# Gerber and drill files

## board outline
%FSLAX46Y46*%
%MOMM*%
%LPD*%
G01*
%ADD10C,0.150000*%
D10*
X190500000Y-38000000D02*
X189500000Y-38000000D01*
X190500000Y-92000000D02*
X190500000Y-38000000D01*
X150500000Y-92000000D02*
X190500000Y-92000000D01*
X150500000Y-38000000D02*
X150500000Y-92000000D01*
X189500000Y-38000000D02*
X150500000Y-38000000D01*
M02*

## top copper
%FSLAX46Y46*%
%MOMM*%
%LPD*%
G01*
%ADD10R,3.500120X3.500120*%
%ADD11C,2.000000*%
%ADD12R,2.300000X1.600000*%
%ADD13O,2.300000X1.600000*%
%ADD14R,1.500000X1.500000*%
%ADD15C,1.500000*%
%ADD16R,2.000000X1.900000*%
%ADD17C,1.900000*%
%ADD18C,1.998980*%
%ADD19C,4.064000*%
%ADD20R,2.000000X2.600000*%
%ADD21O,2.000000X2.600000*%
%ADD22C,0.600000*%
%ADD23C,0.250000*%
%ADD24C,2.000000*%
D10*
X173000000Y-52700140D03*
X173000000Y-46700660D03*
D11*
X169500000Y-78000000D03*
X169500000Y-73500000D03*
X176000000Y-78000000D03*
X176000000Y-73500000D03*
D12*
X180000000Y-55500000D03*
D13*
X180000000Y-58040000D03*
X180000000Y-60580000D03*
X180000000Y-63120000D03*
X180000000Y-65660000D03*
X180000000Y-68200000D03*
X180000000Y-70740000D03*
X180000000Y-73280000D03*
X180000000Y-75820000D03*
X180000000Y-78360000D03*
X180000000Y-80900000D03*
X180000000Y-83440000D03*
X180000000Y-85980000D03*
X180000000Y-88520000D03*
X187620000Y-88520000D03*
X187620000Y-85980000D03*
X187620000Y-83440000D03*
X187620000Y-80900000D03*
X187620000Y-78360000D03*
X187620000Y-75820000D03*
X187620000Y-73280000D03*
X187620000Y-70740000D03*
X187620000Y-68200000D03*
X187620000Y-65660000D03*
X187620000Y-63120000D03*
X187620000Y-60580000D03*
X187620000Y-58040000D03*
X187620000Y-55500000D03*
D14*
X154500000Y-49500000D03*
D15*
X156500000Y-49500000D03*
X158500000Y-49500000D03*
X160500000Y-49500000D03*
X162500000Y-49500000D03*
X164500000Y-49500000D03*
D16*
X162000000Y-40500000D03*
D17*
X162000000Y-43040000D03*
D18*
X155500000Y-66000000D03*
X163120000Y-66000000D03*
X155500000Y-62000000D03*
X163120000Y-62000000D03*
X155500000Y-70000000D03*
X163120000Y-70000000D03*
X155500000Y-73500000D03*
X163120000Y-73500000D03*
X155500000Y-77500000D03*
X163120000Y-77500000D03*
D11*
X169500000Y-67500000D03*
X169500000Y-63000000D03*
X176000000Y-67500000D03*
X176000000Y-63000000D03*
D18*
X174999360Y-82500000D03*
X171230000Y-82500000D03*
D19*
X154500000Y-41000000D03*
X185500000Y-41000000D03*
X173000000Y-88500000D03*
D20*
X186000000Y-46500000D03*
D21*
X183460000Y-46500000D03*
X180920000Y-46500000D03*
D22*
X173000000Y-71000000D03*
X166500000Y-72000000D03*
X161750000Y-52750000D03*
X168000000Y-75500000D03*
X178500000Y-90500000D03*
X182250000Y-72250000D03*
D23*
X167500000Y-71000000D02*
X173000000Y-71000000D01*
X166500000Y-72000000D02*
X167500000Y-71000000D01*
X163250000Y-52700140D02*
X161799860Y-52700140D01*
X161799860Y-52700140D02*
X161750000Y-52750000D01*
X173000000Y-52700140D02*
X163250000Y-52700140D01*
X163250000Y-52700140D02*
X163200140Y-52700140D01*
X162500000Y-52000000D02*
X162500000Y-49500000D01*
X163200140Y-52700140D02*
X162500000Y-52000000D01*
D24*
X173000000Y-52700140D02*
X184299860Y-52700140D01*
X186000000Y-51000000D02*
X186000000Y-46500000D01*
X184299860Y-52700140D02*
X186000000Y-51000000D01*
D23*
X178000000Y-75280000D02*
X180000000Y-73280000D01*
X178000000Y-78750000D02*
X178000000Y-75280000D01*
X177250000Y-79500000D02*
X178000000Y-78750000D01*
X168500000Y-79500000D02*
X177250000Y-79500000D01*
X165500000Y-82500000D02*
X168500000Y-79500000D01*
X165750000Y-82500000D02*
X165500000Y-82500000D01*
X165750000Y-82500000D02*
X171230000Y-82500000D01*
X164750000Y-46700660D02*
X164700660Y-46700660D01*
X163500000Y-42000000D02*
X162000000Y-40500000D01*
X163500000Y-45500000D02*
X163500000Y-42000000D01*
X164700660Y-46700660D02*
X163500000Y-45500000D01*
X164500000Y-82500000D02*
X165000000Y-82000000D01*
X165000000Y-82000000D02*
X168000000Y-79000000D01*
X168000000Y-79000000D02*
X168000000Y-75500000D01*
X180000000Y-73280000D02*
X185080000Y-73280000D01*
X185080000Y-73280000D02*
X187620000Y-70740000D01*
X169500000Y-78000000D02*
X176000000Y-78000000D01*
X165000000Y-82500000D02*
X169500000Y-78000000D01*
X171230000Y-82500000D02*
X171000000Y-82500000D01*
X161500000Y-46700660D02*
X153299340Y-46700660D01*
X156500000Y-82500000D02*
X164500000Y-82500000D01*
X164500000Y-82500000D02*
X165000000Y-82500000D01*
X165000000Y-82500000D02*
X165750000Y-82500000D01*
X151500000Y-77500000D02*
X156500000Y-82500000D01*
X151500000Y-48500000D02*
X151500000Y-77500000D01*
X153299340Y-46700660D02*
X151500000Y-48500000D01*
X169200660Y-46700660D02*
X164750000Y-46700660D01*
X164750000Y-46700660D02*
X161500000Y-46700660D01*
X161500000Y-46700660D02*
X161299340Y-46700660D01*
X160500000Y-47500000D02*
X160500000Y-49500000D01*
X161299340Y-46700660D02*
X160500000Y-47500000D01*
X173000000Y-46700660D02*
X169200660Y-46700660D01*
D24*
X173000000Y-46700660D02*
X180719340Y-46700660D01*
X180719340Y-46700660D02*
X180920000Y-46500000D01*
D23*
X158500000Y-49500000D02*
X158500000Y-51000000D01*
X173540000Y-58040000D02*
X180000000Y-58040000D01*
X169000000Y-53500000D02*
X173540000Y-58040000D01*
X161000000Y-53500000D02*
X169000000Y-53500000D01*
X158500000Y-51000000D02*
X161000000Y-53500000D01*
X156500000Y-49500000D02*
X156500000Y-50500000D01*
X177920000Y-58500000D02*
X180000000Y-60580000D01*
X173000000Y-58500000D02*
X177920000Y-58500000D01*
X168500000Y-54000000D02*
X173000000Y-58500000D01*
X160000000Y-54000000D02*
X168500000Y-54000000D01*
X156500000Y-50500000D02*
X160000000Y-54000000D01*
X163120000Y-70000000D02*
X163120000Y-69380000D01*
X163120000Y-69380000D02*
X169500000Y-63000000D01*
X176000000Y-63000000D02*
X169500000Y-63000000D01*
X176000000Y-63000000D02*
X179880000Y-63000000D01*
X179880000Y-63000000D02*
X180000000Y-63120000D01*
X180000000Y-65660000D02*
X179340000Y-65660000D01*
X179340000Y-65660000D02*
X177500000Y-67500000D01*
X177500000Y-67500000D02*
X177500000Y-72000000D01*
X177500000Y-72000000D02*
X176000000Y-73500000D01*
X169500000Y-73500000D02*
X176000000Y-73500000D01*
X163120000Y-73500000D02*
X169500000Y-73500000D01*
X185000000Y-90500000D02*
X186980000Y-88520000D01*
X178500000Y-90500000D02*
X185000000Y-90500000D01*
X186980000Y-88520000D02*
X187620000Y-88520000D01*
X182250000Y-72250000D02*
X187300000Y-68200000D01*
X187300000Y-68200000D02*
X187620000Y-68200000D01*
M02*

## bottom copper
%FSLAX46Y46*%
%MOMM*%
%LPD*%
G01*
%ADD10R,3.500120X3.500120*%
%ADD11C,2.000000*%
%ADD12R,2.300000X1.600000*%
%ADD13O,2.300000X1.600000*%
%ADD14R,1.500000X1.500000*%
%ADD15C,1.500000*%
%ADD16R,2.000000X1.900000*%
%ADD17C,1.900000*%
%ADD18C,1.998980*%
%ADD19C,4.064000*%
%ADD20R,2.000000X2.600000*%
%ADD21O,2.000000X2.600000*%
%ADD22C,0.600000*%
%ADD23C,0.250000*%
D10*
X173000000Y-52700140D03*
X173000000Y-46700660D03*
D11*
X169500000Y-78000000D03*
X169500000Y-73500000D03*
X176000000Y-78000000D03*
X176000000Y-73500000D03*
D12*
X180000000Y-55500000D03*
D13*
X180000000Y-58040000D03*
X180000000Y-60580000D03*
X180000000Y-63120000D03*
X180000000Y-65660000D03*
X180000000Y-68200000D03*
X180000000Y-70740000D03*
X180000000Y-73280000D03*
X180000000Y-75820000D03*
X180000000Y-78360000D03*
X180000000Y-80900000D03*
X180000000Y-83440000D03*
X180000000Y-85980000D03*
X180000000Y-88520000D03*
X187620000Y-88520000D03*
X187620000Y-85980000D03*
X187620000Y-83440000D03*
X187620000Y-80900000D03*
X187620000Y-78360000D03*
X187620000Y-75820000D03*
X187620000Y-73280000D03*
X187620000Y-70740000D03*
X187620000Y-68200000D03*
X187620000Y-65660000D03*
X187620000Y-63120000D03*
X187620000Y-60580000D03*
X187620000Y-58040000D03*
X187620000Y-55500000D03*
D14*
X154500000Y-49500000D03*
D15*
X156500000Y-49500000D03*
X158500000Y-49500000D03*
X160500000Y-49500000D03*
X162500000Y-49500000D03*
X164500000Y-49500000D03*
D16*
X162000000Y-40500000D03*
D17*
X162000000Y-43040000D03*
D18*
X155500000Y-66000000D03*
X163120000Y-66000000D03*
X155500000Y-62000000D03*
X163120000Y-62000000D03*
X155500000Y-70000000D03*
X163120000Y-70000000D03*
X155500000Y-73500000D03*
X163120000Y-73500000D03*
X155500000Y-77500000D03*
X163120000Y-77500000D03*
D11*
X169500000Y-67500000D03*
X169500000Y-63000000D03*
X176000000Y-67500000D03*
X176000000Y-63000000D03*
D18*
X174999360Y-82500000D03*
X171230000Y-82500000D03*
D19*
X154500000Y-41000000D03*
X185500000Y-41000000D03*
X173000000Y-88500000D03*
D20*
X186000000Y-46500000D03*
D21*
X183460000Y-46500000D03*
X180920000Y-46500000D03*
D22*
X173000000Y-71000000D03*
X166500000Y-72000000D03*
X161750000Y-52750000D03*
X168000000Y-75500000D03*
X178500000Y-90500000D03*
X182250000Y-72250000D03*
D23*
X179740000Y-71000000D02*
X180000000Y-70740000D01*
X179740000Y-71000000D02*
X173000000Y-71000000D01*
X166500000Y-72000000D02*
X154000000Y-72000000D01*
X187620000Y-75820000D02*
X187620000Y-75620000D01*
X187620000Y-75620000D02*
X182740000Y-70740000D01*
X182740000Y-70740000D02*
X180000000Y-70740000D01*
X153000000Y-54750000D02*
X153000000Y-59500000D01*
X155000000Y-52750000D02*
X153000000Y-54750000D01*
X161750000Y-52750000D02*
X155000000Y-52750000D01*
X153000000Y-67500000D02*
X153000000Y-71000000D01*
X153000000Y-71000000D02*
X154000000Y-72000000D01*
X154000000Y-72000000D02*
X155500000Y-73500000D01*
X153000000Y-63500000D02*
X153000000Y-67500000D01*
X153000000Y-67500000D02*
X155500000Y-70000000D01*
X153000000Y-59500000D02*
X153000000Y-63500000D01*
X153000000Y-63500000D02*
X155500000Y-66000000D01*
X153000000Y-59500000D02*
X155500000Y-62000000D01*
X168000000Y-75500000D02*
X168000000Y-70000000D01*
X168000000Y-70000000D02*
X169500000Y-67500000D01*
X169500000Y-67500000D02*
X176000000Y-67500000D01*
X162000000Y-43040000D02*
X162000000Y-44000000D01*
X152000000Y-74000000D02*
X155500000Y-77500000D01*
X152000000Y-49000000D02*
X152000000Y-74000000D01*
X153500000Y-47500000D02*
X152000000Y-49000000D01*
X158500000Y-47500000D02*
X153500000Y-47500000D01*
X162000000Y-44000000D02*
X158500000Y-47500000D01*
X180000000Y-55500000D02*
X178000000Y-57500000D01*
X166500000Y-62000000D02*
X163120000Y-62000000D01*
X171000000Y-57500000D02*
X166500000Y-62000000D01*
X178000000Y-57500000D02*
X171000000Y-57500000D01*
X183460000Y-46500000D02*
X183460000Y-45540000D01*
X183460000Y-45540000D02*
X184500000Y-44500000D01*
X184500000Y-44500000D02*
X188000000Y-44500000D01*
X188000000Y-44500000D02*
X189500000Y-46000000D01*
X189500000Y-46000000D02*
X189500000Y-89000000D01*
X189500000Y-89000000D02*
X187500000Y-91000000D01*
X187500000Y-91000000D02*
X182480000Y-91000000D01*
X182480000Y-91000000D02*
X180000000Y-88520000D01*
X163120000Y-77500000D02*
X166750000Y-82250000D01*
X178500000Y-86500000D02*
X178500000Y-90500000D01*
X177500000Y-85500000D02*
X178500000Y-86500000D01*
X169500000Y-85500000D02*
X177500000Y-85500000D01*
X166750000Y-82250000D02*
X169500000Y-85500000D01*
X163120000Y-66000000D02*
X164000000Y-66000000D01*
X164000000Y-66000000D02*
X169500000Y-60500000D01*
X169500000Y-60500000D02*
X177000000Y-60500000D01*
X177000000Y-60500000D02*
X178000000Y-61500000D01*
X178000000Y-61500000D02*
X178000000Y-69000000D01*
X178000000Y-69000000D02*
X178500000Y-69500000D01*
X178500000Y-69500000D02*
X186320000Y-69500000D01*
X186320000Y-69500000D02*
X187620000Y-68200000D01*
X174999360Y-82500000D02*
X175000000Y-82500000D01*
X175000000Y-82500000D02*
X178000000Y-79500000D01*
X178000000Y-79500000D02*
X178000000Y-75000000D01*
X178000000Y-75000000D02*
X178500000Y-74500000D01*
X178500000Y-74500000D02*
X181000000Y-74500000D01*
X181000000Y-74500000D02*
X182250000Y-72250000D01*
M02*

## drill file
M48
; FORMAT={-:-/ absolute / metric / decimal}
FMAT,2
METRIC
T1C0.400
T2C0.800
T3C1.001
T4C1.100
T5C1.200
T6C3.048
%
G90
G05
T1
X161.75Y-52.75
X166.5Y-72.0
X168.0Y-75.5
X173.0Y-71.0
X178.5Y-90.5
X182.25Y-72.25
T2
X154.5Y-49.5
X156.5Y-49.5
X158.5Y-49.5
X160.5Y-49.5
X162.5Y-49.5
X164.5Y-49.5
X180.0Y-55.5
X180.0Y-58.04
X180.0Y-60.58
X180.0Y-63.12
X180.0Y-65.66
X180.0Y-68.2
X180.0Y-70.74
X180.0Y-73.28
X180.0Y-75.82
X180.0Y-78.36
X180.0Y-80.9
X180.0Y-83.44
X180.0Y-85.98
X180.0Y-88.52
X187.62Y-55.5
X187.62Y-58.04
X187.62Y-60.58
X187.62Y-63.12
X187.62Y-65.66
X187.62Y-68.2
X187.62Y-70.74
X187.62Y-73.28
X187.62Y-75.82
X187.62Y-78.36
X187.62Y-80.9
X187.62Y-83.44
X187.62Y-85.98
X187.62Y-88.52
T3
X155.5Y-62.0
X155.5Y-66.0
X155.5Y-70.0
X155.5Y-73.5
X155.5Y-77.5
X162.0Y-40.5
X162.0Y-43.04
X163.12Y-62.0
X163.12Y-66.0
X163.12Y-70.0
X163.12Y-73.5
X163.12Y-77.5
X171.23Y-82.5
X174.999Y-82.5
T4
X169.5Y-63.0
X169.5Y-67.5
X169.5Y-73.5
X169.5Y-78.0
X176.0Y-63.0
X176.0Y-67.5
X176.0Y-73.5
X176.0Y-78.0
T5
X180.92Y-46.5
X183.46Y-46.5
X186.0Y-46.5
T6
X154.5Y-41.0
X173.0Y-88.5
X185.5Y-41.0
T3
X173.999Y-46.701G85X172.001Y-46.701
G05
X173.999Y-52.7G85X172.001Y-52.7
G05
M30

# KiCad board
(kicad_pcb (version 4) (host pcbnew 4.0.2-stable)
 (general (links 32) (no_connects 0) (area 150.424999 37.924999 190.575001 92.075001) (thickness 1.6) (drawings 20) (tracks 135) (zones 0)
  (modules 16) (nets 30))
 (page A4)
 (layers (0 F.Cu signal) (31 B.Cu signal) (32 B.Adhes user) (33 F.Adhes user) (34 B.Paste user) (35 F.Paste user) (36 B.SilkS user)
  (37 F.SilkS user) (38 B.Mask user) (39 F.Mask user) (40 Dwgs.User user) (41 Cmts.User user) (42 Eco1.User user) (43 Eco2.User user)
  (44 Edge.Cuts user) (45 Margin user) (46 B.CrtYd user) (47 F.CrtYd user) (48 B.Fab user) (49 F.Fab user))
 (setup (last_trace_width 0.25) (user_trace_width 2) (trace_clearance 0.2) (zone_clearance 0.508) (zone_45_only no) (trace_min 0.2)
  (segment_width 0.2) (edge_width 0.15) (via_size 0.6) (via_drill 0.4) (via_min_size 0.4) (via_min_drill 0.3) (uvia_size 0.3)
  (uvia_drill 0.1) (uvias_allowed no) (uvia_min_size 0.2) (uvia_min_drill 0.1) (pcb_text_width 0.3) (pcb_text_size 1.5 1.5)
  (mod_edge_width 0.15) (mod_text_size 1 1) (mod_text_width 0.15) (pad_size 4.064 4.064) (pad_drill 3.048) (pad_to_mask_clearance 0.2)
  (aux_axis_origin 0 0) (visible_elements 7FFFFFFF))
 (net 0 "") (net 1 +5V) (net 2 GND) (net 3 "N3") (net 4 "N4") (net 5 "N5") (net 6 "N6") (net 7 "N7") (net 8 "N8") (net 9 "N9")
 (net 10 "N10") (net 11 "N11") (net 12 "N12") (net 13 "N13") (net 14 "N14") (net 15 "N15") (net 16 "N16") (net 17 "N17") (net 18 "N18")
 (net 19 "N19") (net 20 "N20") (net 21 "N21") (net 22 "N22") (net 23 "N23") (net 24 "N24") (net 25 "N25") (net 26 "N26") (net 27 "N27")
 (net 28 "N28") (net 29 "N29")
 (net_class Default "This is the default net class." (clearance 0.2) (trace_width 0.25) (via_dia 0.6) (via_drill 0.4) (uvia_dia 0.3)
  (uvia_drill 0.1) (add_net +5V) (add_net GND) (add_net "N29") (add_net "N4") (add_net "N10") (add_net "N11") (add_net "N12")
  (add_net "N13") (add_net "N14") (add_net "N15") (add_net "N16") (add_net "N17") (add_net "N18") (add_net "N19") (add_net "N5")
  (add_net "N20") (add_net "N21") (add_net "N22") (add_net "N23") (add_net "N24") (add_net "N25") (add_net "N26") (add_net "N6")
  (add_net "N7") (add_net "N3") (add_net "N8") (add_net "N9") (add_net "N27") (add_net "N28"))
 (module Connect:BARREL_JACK (layer F.Cu) (at 173 46.5 270)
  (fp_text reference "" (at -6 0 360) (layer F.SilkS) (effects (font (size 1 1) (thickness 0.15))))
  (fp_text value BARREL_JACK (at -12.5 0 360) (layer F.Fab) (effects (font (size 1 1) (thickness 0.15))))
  (pad 1 thru_hole rect (at 6.20014 0 270) (size 3.50012 3.50012) (drill oval 1.00076 2.99974) (layers *.Cu *.Mask F.SilkS) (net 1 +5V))
  (pad 2 thru_hole rect (at 0.20066 0 270) (size 3.50012 3.50012) (drill oval 1.00076 2.99974) (layers *.Cu *.Mask F.SilkS) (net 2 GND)))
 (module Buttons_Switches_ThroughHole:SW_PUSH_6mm (layer F.Cu) (at 169.5 73.5)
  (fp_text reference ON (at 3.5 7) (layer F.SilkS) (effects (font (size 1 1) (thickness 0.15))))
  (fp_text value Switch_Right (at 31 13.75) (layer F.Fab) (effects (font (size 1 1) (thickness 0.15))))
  (pad 2 thru_hole circle (at 0 4.5 90) (size 2 2) (drill 1.1) (layers *.Cu *.Mask) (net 2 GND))
  (pad 1 thru_hole circle (at 0 0 90) (size 2 2) (drill 1.1) (layers *.Cu *.Mask) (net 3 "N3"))
  (pad 2 thru_hole circle (at 6.5 4.5 90) (size 2 2) (drill 1.1) (layers *.Cu *.Mask) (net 2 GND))
  (pad 1 thru_hole circle (at 6.5 0 90) (size 2 2) (drill 1.1) (layers *.Cu *.Mask) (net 3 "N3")))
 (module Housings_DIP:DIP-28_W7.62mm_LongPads (layer F.Cu) (at 180 55.5)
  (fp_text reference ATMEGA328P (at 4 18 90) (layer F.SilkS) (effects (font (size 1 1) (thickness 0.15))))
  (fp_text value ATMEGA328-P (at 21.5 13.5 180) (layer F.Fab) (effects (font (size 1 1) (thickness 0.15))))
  (pad 1 thru_hole rect (at 0 0) (size 2.3 1.6) (drill 0.8) (layers *.Cu *.Mask F.SilkS) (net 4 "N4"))
  (pad 2 thru_hole oval (at 0 2.54) (size 2.3 1.6) (drill 0.8) (layers *.Cu *.Mask F.SilkS) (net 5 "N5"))
  (pad 3 thru_hole oval (at 0 5.08) (size 2.3 1.6) (drill 0.8) (layers *.Cu *.Mask F.SilkS) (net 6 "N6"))
  (pad 4 thru_hole oval (at 0 7.62) (size 2.3 1.6) (drill 0.8) (layers *.Cu *.Mask F.SilkS) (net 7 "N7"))
  (pad 5 thru_hole oval (at 0 10.16) (size 2.3 1.6) (drill 0.8) (layers *.Cu *.Mask F.SilkS) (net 3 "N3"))
  (pad 6 thru_hole oval (at 0 12.7) (size 2.3 1.6) (drill 0.8) (layers *.Cu *.Mask F.SilkS) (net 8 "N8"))
  (pad 7 thru_hole oval (at 0 15.24) (size 2.3 1.6) (drill 0.8) (layers *.Cu *.Mask F.SilkS) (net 1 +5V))
  (pad 8 thru_hole oval (at 0 17.78) (size 2.3 1.6) (drill 0.8) (layers *.Cu *.Mask F.SilkS) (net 2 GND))
  (pad 9 thru_hole oval (at 0 20.32) (size 2.3 1.6) (drill 0.8) (layers *.Cu *.Mask F.SilkS) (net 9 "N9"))
  (pad 10 thru_hole oval (at 0 22.86) (size 2.3 1.6) (drill 0.8) (layers *.Cu *.Mask F.SilkS) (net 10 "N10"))
  (pad 11 thru_hole oval (at 0 25.4) (size 2.3 1.6) (drill 0.8) (layers *.Cu *.Mask F.SilkS) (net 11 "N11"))
  (pad 12 thru_hole oval (at 0 27.94) (size 2.3 1.6) (drill 0.8) (layers *.Cu *.Mask F.SilkS) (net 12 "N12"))
  (pad 13 thru_hole oval (at 0 30.48) (size 2.3 1.6) (drill 0.8) (layers *.Cu *.Mask F.SilkS) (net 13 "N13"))
  (pad 14 thru_hole oval (at 0 33.02) (size 2.3 1.6) (drill 0.8) (layers *.Cu *.Mask F.SilkS) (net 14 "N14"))
  (pad 15 thru_hole oval (at 7.62 33.02) (size 2.3 1.6) (drill 0.8) (layers *.Cu *.Mask F.SilkS) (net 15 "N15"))
  (pad 16 thru_hole oval (at 7.62 30.48) (size 2.3 1.6) (drill 0.8) (layers *.Cu *.Mask F.SilkS) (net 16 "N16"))
  (pad 17 thru_hole oval (at 7.62 27.94) (size 2.3 1.6) (drill 0.8) (layers *.Cu *.Mask F.SilkS) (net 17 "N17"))
  (pad 18 thru_hole oval (at 7.62 25.4) (size 2.3 1.6) (drill 0.8) (layers *.Cu *.Mask F.SilkS) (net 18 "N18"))
  (pad 19 thru_hole oval (at 7.62 22.86) (size 2.3 1.6) (drill 0.8) (layers *.Cu *.Mask F.SilkS) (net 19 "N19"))
  (pad 20 thru_hole oval (at 7.62 20.32) (size 2.3 1.6) (drill 0.8) (layers *.Cu *.Mask F.SilkS) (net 1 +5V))
  (pad 21 thru_hole oval (at 7.62 17.78) (size 2.3 1.6) (drill 0.8) (layers *.Cu *.Mask F.SilkS) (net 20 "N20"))
  (pad 22 thru_hole oval (at 7.62 15.24) (size 2.3 1.6) (drill 0.8) (layers *.Cu *.Mask F.SilkS) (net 2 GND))
  (pad 23 thru_hole oval (at 7.62 12.7) (size 2.3 1.6) (drill 0.8) (layers *.Cu *.Mask F.SilkS) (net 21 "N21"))
  (pad 24 thru_hole oval (at 7.62 10.16) (size 2.3 1.6) (drill 0.8) (layers *.Cu *.Mask F.SilkS) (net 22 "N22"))
  (pad 25 thru_hole oval (at 7.62 7.62) (size 2.3 1.6) (drill 0.8) (layers *.Cu *.Mask F.SilkS) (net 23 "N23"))
  (pad 26 thru_hole oval (at 7.62 5.08) (size 2.3 1.6) (drill 0.8) (layers *.Cu *.Mask F.SilkS) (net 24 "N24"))
  (pad 27 thru_hole oval (at 7.62 2.54) (size 2.3 1.6) (drill 0.8) (layers *.Cu *.Mask F.SilkS) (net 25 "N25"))
  (pad 28 thru_hole oval (at 7.62 0) (size 2.3 1.6) (drill 0.8) (layers *.Cu *.Mask F.SilkS) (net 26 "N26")))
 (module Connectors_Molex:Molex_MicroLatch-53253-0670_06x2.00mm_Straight (layer F.Cu) (at 154.5 49.5)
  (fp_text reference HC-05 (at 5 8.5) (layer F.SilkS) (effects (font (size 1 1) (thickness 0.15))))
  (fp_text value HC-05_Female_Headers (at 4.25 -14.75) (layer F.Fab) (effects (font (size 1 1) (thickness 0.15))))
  (pad 1 thru_hole rect (at 0 0) (size 1.5 1.5) (drill 0.8) (layers *.Cu *.Mask) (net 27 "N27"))
  (pad 2 thru_hole circle (at 2 0) (size 1.5 1.5) (drill 0.8) (layers *.Cu *.Mask) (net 6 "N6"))
  (pad 3 thru_hole circle (at 4 0) (size 1.5 1.5) (drill 0.8) (layers *.Cu *.Mask) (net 5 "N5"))
  (pad 4 thru_hole circle (at 6 0) (size 1.5 1.5) (drill 0.8) (layers *.Cu *.Mask) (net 2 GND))
  (pad 5 thru_hole circle (at 8 0) (size 1.5 1.5) (drill 0.8) (layers *.Cu *.Mask) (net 1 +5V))
  (pad 6 thru_hole circle (at 10 0) (size 1.5 1.5) (drill 0.8) (layers *.Cu *.Mask) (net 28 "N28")))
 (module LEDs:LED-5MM (layer F.Cu) (at 162 40.5 270)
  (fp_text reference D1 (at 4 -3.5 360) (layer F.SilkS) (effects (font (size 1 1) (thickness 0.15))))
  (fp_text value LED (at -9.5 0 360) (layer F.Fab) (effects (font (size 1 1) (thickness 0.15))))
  (pad 1 thru_hole rect (at 0 0) (size 2 1.9) (drill 1.00076) (layers *.Cu *.Mask F.SilkS) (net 2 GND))
  (pad 2 thru_hole circle (at 2.54 0 270) (size 1.9 1.9) (drill 1.00076) (layers *.Cu *.Mask F.SilkS) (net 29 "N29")))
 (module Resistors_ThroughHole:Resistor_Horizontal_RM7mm (layer F.Cu) (at 155.5 66)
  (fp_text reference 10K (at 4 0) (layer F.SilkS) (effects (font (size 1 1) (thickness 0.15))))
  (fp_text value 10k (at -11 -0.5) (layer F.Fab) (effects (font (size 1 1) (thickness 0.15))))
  (pad 1 thru_hole circle (at 0 0) (size 1.99898 1.99898) (drill 1.00076) (layers *.Cu *.SilkS *.Mask) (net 1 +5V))
  (pad 2 thru_hole circle (at 7.62 0) (size 1.99898 1.99898) (drill 1.00076) (layers *.Cu *.SilkS *.Mask) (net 21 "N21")))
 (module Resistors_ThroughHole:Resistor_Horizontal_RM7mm (layer F.Cu) (at 155.5 62)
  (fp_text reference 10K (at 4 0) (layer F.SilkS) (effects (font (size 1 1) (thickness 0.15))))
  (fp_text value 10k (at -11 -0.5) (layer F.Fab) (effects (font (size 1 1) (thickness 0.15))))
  (pad 1 thru_hole circle (at 0 0) (size 1.99898 1.99898) (drill 1.00076) (layers *.Cu *.SilkS *.Mask) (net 1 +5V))
  (pad 2 thru_hole circle (at 7.62 0) (size 1.99898 1.99898) (drill 1.00076) (layers *.Cu *.SilkS *.Mask) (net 4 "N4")))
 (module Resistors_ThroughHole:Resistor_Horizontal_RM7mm (layer F.Cu) (at 155.5 70)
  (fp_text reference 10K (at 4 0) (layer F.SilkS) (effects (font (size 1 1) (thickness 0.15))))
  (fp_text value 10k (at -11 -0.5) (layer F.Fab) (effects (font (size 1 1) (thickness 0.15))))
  (pad 1 thru_hole circle (at 0 0) (size 1.99898 1.99898) (drill 1.00076) (layers *.Cu *.SilkS *.Mask) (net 1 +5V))
  (pad 2 thru_hole circle (at 7.62 0) (size 1.99898 1.99898) (drill 1.00076) (layers *.Cu *.SilkS *.Mask) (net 7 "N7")))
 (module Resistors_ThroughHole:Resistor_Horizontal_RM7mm (layer F.Cu) (at 155.5 73.5)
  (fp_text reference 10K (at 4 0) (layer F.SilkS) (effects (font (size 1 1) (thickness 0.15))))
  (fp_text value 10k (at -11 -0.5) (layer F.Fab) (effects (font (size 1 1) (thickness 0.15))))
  (pad 1 thru_hole circle (at 0 0) (size 1.99898 1.99898) (drill 1.00076) (layers *.Cu *.SilkS *.Mask) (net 1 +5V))
  (pad 2 thru_hole circle (at 7.62 0) (size 1.99898 1.99898) (drill 1.00076) (layers *.Cu *.SilkS *.Mask) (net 3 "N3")))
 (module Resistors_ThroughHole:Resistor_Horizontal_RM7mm (layer F.Cu) (at 155.5 77.5)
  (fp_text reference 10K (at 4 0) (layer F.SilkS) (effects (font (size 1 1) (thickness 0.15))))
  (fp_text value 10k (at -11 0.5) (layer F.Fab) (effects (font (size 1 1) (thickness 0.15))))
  (pad 1 thru_hole circle (at 0 0) (size 1.99898 1.99898) (drill 1.00076) (layers *.Cu *.SilkS *.Mask) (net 29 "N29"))
  (pad 2 thru_hole circle (at 7.62 0) (size 1.99898 1.99898) (drill 1.00076) (layers *.Cu *.SilkS *.Mask) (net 15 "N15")))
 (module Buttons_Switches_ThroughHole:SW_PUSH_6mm (layer F.Cu) (at 169.5 63)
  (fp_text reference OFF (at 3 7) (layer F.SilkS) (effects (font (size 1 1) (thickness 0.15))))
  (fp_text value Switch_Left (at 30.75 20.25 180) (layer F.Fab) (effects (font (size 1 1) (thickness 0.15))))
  (pad 2 thru_hole circle (at 0 4.5 90) (size 2 2) (drill 1.1) (layers *.Cu *.Mask) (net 2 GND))
  (pad 1 thru_hole circle (at 0 0 90) (size 2 2) (drill 1.1) (layers *.Cu *.Mask) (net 7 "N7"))
  (pad 2 thru_hole circle (at 6.5 4.5 90) (size 2 2) (drill 1.1) (layers *.Cu *.Mask) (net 2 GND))
  (pad 1 thru_hole circle (at 6.5 0 90) (size 2 2) (drill 1.1) (layers *.Cu *.Mask) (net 7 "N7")))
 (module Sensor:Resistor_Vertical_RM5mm (layer F.Cu) (at 172.5 82.5 180)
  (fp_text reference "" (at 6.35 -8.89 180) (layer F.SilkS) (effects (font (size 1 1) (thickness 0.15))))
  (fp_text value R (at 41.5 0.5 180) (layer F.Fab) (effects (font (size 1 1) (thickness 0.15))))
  (pad 1 thru_hole circle (at -2.49936 0 180) (size 1.99898 1.99898) (drill 1.00076) (layers *.Cu *.Mask B.SilkS) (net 21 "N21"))
  (pad 2 thru_hole circle (at 1.27 0 180) (size 1.99898 1.99898) (drill 1.00076) (layers *.Cu *.SilkS *.Mask) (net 2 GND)))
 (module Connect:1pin (layer F.Cu) (at 154.5 41)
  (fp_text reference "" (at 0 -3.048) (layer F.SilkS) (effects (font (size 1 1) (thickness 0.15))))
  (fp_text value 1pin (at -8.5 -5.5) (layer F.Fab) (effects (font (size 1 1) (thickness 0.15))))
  (pad 1 thru_hole circle (at 0 0) (size 4.064 4.064) (drill 3.048) (layers *.Cu *.Mask F.SilkS)))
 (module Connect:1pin (layer F.Cu) (at 185.5 41)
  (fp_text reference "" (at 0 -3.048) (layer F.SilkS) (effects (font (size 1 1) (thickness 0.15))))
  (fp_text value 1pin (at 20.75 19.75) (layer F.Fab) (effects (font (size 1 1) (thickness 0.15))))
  (pad 1 thru_hole circle (at 0 0) (size 4.064 4.064) (drill 3.048) (layers *.Cu *.Mask F.SilkS)))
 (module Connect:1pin (layer F.Cu) (at 173 88.5)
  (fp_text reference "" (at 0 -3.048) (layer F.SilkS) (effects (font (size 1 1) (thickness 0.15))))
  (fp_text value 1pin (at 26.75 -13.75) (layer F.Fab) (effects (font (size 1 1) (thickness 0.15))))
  (pad 1 thru_hole circle (at 0 0) (size 4.064 4.064) (drill 3.048) (layers *.Cu *.Mask F.SilkS)))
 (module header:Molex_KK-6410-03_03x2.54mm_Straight (layer F.Cu) (at 186 46.5 180)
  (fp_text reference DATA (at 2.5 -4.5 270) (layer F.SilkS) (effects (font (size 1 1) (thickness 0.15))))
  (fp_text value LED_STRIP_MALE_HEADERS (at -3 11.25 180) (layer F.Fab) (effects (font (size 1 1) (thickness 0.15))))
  (pad 1 thru_hole rect (at 0 0 180) (size 2 2.6) (drill 1.2) (layers *.Cu *.Mask F.SilkS) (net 1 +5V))
  (pad 2 thru_hole oval (at 2.54 0 180) (size 2 2.6) (drill 1.2) (layers *.Cu *.Mask F.SilkS) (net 14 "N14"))
  (pad 3 thru_hole oval (at 5.08 0 180) (size 2 2.6) (drill 1.2) (layers *.Cu *.Mask F.SilkS) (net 2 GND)))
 (gr_line (start 190.5 38) (end 189.5 38) (angle 90) (layer Edge.Cuts) (width 0.15))
 (gr_line (start 190.5 92) (end 190.5 38) (angle 90) (layer Edge.Cuts) (width 0.15))
 (gr_line (start 150.5 92) (end 190.5 92) (angle 90) (layer Edge.Cuts) (width 0.15))
 (gr_line (start 150.5 38) (end 150.5 92) (angle 90) (layer Edge.Cuts) (width 0.15))
 (gr_line (start 189.5 38) (end 150.5 38) (angle 90) (layer Edge.Cuts) (width 0.15))
 (segment (start 179.74 71) (end 180 70.74) (width 0.25) (layer B.Cu) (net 1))
 (segment (start 179.74 71) (end 173 71) (width 0.25) (layer B.Cu) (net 1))
 (segment (start 166.5 72) (end 154 72) (width 0.25) (layer B.Cu) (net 1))
 (via (at 173 71) (size 0.6) (drill 0.4) (layers F.Cu B.Cu) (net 1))
 (segment (start 167.5 71) (end 173 71) (width 0.25) (layer F.Cu) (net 1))
 (segment (start 166.5 72) (end 167.5 71) (width 0.25) (layer F.Cu) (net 1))
 (via (at 166.5 72) (size 0.6) (drill 0.4) (layers F.Cu B.Cu) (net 1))
 (segment (start 187.62 75.82) (end 187.62 75.62) (width 0.25) (layer B.Cu) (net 1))
 (segment (start 187.62 75.62) (end 182.74 70.74) (width 0.25) (layer B.Cu) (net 1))
 (segment (start 182.74 70.74) (end 180 70.74) (width 0.25) (layer B.Cu) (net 1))
 (segment (start 163.25 52.70014) (end 161.79986 52.70014) (width 0.25) (layer F.Cu) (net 1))
 (segment (start 153 54.75) (end 153 59.5) (width 0.25) (layer B.Cu) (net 1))
 (segment (start 155 52.75) (end 153 54.75) (width 0.25) (layer B.Cu) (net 1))
 (segment (start 161.75 52.75) (end 155 52.75) (width 0.25) (layer B.Cu) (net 1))
 (via (at 161.75 52.75) (size 0.6) (drill 0.4) (layers F.Cu B.Cu) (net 1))
 (segment (start 161.79986 52.70014) (end 161.75 52.75) (width 0.25) (layer F.Cu) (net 1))
 (segment (start 173 52.70014) (end 163.25 52.70014) (width 0.25) (layer F.Cu) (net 1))
 (segment (start 163.25 52.70014) (end 163.20014 52.70014) (width 0.25) (layer F.Cu) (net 1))
 (segment (start 162.5 52) (end 162.5 49.5) (width 0.25) (layer F.Cu) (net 1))
 (segment (start 163.20014 52.70014) (end 162.5 52) (width 0.25) (layer F.Cu) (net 1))
 (segment (start 153 67.5) (end 153 71) (width 0.25) (layer B.Cu) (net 1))
 (segment (start 153 71) (end 154 72) (width 0.25) (layer B.Cu) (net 1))
 (segment (start 154 72) (end 155.5 73.5) (width 0.25) (layer B.Cu) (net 1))
 (segment (start 153 63.5) (end 153 67.5) (width 0.25) (layer B.Cu) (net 1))
 (segment (start 153 67.5) (end 155.5 70) (width 0.25) (layer B.Cu) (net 1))
 (segment (start 153 59.5) (end 153 63.5) (width 0.25) (layer B.Cu) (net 1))
 (segment (start 153 63.5) (end 155.5 66) (width 0.25) (layer B.Cu) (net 1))
 (segment (start 153 59.5) (end 155.5 62) (width 0.25) (layer B.Cu) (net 1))
 (segment (start 173 52.70014) (end 184.29986 52.70014) (width 2) (layer F.Cu) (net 1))
 (segment (start 186 51) (end 186 46.5) (width 2) (layer F.Cu) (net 1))
 (segment (start 184.29986 52.70014) (end 186 51) (width 2) (layer F.Cu) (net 1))
 (segment (start 178 75.28) (end 180 73.28) (width 0.25) (layer F.Cu) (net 2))
 (segment (start 178 78.75) (end 178 75.28) (width 0.25) (layer F.Cu) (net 2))
 (segment (start 177.25 79.5) (end 178 78.75) (width 0.25) (layer F.Cu) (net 2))
 (segment (start 168.5 79.5) (end 177.25 79.5) (width 0.25) (layer F.Cu) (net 2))
 (segment (start 165.5 82.5) (end 168.5 79.5) (width 0.25) (layer F.Cu) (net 2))
 (segment (start 165.75 82.5) (end 165.5 82.5) (width 0.25) (layer F.Cu) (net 2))
 (segment (start 165.75 82.5) (end 171.23 82.5) (width 0.25) (layer F.Cu) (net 2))
 (segment (start 164.75 46.70066) (end 164.70066 46.70066) (width 0.25) (layer F.Cu) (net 2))
 (segment (start 163.5 42) (end 162 40.5) (width 0.25) (layer F.Cu) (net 2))
 (segment (start 163.5 45.5) (end 163.5 42) (width 0.25) (layer F.Cu) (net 2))
 (segment (start 164.70066 46.70066) (end 163.5 45.5) (width 0.25) (layer F.Cu) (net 2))
 (segment (start 164.5 82.5) (end 165 82) (width 0.25) (layer F.Cu) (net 2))
 (segment (start 165 82) (end 168 79) (width 0.25) (layer F.Cu) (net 2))
 (segment (start 168 79) (end 168 75.5) (width 0.25) (layer F.Cu) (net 2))
 (via (at 168 75.5) (size 0.6) (drill 0.4) (layers F.Cu B.Cu) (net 2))
 (segment (start 168 75.5) (end 168 70) (width 0.25) (layer B.Cu) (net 2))
 (segment (start 168 70) (end 169.5 67.5) (width 0.25) (layer B.Cu) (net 2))
 (segment (start 180 73.28) (end 185.08 73.28) (width 0.25) (layer F.Cu) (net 2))
 (segment (start 185.08 73.28) (end 187.62 70.74) (width 0.25) (layer F.Cu) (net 2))
 (segment (start 169.5 67.5) (end 176 67.5) (width 0.25) (layer B.Cu) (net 2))
 (segment (start 169.5 78) (end 176 78) (width 0.25) (layer F.Cu) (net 2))
 (segment (start 165 82.5) (end 169.5 78) (width 0.25) (layer F.Cu) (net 2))
 (segment (start 171.23 82.5) (end 171 82.5) (width 0.25) (layer F.Cu) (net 2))
 (segment (start 161.5 46.70066) (end 153.29934 46.70066) (width 0.25) (layer F.Cu) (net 2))
 (segment (start 156.5 82.5) (end 164.5 82.5) (width 0.25) (layer F.Cu) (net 2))
 (segment (start 164.5 82.5) (end 165 82.5) (width 0.25) (layer F.Cu) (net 2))
 (segment (start 165 82.5) (end 165.75 82.5) (width 0.25) (layer F.Cu) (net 2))
 (segment (start 151.5 77.5) (end 156.5 82.5) (width 0.25) (layer F.Cu) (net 2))
 (segment (start 151.5 48.5) (end 151.5 77.5) (width 0.25) (layer F.Cu) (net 2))
 (segment (start 153.29934 46.70066) (end 151.5 48.5) (width 0.25) (layer F.Cu) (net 2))
 (segment (start 169.20066 46.70066) (end 164.75 46.70066) (width 0.25) (layer F.Cu) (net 2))
 (segment (start 164.75 46.70066) (end 161.5 46.70066) (width 0.25) (layer F.Cu) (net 2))
 (segment (start 161.5 46.70066) (end 161.29934 46.70066) (width 0.25) (layer F.Cu) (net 2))
 (segment (start 160.5 47.5) (end 160.5 49.5) (width 0.25) (layer F.Cu) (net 2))
 (segment (start 161.29934 46.70066) (end 160.5 47.5) (width 0.25) (layer F.Cu) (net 2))
 (segment (start 173 46.70066) (end 169.20066 46.70066) (width 0.25) (layer F.Cu) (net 2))
 (segment (start 173 46.70066) (end 180.71934 46.70066) (width 2) (layer F.Cu) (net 2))
 (segment (start 180.71934 46.70066) (end 180.92 46.5) (width 2) (layer F.Cu) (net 2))
 (segment (start 162 43.04) (end 162 44) (width 0.25) (layer B.Cu) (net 29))
 (segment (start 152 74) (end 155.5 77.5) (width 0.25) (layer B.Cu) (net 29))
 (segment (start 152 49) (end 152 74) (width 0.25) (layer B.Cu) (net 29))
 (segment (start 153.5 47.5) (end 152 49) (width 0.25) (layer B.Cu) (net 29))
 (segment (start 158.5 47.5) (end 153.5 47.5) (width 0.25) (layer B.Cu) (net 29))
 (segment (start 162 44) (end 158.5 47.5) (width 0.25) (layer B.Cu) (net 29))
 (segment (start 180 55.5) (end 178 57.5) (width 0.25) (layer B.Cu) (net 4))
 (segment (start 166.5 62) (end 163.12 62) (width 0.25) (layer B.Cu) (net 4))
 (segment (start 171 57.5) (end 166.5 62) (width 0.25) (layer B.Cu) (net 4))
 (segment (start 178 57.5) (end 171 57.5) (width 0.25) (layer B.Cu) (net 4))
 (segment (start 158.5 49.5) (end 158.5 51) (width 0.25) (layer F.Cu) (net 5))
 (segment (start 173.54 58.04) (end 180 58.04) (width 0.25) (layer F.Cu) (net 5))
 (segment (start 169 53.5) (end 173.54 58.04) (width 0.25) (layer F.Cu) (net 5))
 (segment (start 161 53.5) (end 169 53.5) (width 0.25) (layer F.Cu) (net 5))
 (segment (start 158.5 51) (end 161 53.5) (width 0.25) (layer F.Cu) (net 5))
 (segment (start 156.5 49.5) (end 156.5 50.5) (width 0.25) (layer F.Cu) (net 6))
 (segment (start 177.92 58.5) (end 180 60.58) (width 0.25) (layer F.Cu) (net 6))
 (segment (start 173 58.5) (end 177.92 58.5) (width 0.25) (layer F.Cu) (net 6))
 (segment (start 168.5 54) (end 173 58.5) (width 0.25) (layer F.Cu) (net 6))
 (segment (start 160 54) (end 168.5 54) (width 0.25) (layer F.Cu) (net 6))
 (segment (start 156.5 50.5) (end 160 54) (width 0.25) (layer F.Cu) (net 6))
 (segment (start 163.12 70) (end 163.12 69.38) (width 0.25) (layer F.Cu) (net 7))
 (segment (start 163.12 69.38) (end 169.5 63) (width 0.25) (layer F.Cu) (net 7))
 (segment (start 176 63) (end 169.5 63) (width 0.25) (layer F.Cu) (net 7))
 (segment (start 176 63) (end 179.88 63) (width 0.25) (layer F.Cu) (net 7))
 (segment (start 179.88 63) (end 180 63.12) (width 0.25) (layer F.Cu) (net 7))
 (segment (start 180 65.66) (end 179.34 65.66) (width 0.25) (layer F.Cu) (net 3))
 (segment (start 179.34 65.66) (end 177.5 67.5) (width 0.25) (layer F.Cu) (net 3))
 (segment (start 177.5 67.5) (end 177.5 72) (width 0.25) (layer F.Cu) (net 3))
 (segment (start 177.5 72) (end 176 73.5) (width 0.25) (layer F.Cu) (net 3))
 (segment (start 169.5 73.5) (end 176 73.5) (width 0.25) (layer F.Cu) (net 3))
 (segment (start 163.12 73.5) (end 169.5 73.5) (width 0.25) (layer F.Cu) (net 3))
 (segment (start 183.46 46.5) (end 183.46 45.54) (width 0.25) (layer B.Cu) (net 14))
 (segment (start 183.46 45.54) (end 184.5 44.5) (width 0.25) (layer B.Cu) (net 14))
 (segment (start 184.5 44.5) (end 188 44.5) (width 0.25) (layer B.Cu) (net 14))
 (segment (start 188 44.5) (end 189.5 46) (width 0.25) (layer B.Cu) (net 14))
 (segment (start 189.5 46) (end 189.5 89) (width 0.25) (layer B.Cu) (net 14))
 (segment (start 189.5 89) (end 187.5 91) (width 0.25) (layer B.Cu) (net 14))
 (segment (start 187.5 91) (end 182.48 91) (width 0.25) (layer B.Cu) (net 14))
 (segment (start 182.48 91) (end 180 88.52) (width 0.25) (layer B.Cu) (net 14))
 (segment (start 163.12 77.5) (end 166.75 82.25) (width 0.25) (layer B.Cu) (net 15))
 (segment (start 185 90.5) (end 186.98 88.52) (width 0.25) (layer F.Cu) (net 15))
 (segment (start 178.5 90.5) (end 185 90.5) (width 0.25) (layer F.Cu) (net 15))
 (via (at 178.5 90.5) (size 0.6) (drill 0.4) (layers F.Cu B.Cu) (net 15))
 (segment (start 178.5 86.5) (end 178.5 90.5) (width 0.25) (layer B.Cu) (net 15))
 (segment (start 177.5 85.5) (end 178.5 86.5) (width 0.25) (layer B.Cu) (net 15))
 (segment (start 169.5 85.5) (end 177.5 85.5) (width 0.25) (layer B.Cu) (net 15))
 (segment (start 166.75 82.25) (end 169.5 85.5) (width 0.25) (layer B.Cu) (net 15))
 (segment (start 186.98 88.52) (end 187.62 88.52) (width 0.25) (layer F.Cu) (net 15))
 (segment (start 163.12 66) (end 164 66) (width 0.25) (layer B.Cu) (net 21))
 (segment (start 164 66) (end 169.5 60.5) (width 0.25) (layer B.Cu) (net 21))
 (segment (start 169.5 60.5) (end 177 60.5) (width 0.25) (layer B.Cu) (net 21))
 (segment (start 177 60.5) (end 178 61.5) (width 0.25) (layer B.Cu) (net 21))
 (segment (start 178 61.5) (end 178 69) (width 0.25) (layer B.Cu) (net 21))
 (segment (start 178 69) (end 178.5 69.5) (width 0.25) (layer B.Cu) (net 21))
 (segment (start 178.5 69.5) (end 186.32 69.5) (width 0.25) (layer B.Cu) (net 21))
 (segment (start 186.32 69.5) (end 187.62 68.2) (width 0.25) (layer B.Cu) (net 21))
 (segment (start 174.99936 82.5) (end 175 82.5) (width 0.25) (layer B.Cu) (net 21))
 (segment (start 175 82.5) (end 178 79.5) (width 0.25) (layer B.Cu) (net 21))
 (segment (start 178 79.5) (end 178 75) (width 0.25) (layer B.Cu) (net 21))
 (segment (start 178 75) (end 178.5 74.5) (width 0.25) (layer B.Cu) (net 21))
 (segment (start 178.5 74.5) (end 181 74.5) (width 0.25) (layer B.Cu) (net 21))
 (segment (start 181 74.5) (end 182.25 72.25) (width 0.25) (layer B.Cu) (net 21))
 (via (at 182.25 72.25) (size 0.6) (drill 0.4) (layers F.Cu B.Cu) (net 21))
 (segment (start 182.25 72.25) (end 187.3 68.2) (width 0.25) (layer F.Cu) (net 21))
 (segment (start 187.3 68.2) (end 187.62 68.2) (width 0.25) (layer F.Cu) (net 21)))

